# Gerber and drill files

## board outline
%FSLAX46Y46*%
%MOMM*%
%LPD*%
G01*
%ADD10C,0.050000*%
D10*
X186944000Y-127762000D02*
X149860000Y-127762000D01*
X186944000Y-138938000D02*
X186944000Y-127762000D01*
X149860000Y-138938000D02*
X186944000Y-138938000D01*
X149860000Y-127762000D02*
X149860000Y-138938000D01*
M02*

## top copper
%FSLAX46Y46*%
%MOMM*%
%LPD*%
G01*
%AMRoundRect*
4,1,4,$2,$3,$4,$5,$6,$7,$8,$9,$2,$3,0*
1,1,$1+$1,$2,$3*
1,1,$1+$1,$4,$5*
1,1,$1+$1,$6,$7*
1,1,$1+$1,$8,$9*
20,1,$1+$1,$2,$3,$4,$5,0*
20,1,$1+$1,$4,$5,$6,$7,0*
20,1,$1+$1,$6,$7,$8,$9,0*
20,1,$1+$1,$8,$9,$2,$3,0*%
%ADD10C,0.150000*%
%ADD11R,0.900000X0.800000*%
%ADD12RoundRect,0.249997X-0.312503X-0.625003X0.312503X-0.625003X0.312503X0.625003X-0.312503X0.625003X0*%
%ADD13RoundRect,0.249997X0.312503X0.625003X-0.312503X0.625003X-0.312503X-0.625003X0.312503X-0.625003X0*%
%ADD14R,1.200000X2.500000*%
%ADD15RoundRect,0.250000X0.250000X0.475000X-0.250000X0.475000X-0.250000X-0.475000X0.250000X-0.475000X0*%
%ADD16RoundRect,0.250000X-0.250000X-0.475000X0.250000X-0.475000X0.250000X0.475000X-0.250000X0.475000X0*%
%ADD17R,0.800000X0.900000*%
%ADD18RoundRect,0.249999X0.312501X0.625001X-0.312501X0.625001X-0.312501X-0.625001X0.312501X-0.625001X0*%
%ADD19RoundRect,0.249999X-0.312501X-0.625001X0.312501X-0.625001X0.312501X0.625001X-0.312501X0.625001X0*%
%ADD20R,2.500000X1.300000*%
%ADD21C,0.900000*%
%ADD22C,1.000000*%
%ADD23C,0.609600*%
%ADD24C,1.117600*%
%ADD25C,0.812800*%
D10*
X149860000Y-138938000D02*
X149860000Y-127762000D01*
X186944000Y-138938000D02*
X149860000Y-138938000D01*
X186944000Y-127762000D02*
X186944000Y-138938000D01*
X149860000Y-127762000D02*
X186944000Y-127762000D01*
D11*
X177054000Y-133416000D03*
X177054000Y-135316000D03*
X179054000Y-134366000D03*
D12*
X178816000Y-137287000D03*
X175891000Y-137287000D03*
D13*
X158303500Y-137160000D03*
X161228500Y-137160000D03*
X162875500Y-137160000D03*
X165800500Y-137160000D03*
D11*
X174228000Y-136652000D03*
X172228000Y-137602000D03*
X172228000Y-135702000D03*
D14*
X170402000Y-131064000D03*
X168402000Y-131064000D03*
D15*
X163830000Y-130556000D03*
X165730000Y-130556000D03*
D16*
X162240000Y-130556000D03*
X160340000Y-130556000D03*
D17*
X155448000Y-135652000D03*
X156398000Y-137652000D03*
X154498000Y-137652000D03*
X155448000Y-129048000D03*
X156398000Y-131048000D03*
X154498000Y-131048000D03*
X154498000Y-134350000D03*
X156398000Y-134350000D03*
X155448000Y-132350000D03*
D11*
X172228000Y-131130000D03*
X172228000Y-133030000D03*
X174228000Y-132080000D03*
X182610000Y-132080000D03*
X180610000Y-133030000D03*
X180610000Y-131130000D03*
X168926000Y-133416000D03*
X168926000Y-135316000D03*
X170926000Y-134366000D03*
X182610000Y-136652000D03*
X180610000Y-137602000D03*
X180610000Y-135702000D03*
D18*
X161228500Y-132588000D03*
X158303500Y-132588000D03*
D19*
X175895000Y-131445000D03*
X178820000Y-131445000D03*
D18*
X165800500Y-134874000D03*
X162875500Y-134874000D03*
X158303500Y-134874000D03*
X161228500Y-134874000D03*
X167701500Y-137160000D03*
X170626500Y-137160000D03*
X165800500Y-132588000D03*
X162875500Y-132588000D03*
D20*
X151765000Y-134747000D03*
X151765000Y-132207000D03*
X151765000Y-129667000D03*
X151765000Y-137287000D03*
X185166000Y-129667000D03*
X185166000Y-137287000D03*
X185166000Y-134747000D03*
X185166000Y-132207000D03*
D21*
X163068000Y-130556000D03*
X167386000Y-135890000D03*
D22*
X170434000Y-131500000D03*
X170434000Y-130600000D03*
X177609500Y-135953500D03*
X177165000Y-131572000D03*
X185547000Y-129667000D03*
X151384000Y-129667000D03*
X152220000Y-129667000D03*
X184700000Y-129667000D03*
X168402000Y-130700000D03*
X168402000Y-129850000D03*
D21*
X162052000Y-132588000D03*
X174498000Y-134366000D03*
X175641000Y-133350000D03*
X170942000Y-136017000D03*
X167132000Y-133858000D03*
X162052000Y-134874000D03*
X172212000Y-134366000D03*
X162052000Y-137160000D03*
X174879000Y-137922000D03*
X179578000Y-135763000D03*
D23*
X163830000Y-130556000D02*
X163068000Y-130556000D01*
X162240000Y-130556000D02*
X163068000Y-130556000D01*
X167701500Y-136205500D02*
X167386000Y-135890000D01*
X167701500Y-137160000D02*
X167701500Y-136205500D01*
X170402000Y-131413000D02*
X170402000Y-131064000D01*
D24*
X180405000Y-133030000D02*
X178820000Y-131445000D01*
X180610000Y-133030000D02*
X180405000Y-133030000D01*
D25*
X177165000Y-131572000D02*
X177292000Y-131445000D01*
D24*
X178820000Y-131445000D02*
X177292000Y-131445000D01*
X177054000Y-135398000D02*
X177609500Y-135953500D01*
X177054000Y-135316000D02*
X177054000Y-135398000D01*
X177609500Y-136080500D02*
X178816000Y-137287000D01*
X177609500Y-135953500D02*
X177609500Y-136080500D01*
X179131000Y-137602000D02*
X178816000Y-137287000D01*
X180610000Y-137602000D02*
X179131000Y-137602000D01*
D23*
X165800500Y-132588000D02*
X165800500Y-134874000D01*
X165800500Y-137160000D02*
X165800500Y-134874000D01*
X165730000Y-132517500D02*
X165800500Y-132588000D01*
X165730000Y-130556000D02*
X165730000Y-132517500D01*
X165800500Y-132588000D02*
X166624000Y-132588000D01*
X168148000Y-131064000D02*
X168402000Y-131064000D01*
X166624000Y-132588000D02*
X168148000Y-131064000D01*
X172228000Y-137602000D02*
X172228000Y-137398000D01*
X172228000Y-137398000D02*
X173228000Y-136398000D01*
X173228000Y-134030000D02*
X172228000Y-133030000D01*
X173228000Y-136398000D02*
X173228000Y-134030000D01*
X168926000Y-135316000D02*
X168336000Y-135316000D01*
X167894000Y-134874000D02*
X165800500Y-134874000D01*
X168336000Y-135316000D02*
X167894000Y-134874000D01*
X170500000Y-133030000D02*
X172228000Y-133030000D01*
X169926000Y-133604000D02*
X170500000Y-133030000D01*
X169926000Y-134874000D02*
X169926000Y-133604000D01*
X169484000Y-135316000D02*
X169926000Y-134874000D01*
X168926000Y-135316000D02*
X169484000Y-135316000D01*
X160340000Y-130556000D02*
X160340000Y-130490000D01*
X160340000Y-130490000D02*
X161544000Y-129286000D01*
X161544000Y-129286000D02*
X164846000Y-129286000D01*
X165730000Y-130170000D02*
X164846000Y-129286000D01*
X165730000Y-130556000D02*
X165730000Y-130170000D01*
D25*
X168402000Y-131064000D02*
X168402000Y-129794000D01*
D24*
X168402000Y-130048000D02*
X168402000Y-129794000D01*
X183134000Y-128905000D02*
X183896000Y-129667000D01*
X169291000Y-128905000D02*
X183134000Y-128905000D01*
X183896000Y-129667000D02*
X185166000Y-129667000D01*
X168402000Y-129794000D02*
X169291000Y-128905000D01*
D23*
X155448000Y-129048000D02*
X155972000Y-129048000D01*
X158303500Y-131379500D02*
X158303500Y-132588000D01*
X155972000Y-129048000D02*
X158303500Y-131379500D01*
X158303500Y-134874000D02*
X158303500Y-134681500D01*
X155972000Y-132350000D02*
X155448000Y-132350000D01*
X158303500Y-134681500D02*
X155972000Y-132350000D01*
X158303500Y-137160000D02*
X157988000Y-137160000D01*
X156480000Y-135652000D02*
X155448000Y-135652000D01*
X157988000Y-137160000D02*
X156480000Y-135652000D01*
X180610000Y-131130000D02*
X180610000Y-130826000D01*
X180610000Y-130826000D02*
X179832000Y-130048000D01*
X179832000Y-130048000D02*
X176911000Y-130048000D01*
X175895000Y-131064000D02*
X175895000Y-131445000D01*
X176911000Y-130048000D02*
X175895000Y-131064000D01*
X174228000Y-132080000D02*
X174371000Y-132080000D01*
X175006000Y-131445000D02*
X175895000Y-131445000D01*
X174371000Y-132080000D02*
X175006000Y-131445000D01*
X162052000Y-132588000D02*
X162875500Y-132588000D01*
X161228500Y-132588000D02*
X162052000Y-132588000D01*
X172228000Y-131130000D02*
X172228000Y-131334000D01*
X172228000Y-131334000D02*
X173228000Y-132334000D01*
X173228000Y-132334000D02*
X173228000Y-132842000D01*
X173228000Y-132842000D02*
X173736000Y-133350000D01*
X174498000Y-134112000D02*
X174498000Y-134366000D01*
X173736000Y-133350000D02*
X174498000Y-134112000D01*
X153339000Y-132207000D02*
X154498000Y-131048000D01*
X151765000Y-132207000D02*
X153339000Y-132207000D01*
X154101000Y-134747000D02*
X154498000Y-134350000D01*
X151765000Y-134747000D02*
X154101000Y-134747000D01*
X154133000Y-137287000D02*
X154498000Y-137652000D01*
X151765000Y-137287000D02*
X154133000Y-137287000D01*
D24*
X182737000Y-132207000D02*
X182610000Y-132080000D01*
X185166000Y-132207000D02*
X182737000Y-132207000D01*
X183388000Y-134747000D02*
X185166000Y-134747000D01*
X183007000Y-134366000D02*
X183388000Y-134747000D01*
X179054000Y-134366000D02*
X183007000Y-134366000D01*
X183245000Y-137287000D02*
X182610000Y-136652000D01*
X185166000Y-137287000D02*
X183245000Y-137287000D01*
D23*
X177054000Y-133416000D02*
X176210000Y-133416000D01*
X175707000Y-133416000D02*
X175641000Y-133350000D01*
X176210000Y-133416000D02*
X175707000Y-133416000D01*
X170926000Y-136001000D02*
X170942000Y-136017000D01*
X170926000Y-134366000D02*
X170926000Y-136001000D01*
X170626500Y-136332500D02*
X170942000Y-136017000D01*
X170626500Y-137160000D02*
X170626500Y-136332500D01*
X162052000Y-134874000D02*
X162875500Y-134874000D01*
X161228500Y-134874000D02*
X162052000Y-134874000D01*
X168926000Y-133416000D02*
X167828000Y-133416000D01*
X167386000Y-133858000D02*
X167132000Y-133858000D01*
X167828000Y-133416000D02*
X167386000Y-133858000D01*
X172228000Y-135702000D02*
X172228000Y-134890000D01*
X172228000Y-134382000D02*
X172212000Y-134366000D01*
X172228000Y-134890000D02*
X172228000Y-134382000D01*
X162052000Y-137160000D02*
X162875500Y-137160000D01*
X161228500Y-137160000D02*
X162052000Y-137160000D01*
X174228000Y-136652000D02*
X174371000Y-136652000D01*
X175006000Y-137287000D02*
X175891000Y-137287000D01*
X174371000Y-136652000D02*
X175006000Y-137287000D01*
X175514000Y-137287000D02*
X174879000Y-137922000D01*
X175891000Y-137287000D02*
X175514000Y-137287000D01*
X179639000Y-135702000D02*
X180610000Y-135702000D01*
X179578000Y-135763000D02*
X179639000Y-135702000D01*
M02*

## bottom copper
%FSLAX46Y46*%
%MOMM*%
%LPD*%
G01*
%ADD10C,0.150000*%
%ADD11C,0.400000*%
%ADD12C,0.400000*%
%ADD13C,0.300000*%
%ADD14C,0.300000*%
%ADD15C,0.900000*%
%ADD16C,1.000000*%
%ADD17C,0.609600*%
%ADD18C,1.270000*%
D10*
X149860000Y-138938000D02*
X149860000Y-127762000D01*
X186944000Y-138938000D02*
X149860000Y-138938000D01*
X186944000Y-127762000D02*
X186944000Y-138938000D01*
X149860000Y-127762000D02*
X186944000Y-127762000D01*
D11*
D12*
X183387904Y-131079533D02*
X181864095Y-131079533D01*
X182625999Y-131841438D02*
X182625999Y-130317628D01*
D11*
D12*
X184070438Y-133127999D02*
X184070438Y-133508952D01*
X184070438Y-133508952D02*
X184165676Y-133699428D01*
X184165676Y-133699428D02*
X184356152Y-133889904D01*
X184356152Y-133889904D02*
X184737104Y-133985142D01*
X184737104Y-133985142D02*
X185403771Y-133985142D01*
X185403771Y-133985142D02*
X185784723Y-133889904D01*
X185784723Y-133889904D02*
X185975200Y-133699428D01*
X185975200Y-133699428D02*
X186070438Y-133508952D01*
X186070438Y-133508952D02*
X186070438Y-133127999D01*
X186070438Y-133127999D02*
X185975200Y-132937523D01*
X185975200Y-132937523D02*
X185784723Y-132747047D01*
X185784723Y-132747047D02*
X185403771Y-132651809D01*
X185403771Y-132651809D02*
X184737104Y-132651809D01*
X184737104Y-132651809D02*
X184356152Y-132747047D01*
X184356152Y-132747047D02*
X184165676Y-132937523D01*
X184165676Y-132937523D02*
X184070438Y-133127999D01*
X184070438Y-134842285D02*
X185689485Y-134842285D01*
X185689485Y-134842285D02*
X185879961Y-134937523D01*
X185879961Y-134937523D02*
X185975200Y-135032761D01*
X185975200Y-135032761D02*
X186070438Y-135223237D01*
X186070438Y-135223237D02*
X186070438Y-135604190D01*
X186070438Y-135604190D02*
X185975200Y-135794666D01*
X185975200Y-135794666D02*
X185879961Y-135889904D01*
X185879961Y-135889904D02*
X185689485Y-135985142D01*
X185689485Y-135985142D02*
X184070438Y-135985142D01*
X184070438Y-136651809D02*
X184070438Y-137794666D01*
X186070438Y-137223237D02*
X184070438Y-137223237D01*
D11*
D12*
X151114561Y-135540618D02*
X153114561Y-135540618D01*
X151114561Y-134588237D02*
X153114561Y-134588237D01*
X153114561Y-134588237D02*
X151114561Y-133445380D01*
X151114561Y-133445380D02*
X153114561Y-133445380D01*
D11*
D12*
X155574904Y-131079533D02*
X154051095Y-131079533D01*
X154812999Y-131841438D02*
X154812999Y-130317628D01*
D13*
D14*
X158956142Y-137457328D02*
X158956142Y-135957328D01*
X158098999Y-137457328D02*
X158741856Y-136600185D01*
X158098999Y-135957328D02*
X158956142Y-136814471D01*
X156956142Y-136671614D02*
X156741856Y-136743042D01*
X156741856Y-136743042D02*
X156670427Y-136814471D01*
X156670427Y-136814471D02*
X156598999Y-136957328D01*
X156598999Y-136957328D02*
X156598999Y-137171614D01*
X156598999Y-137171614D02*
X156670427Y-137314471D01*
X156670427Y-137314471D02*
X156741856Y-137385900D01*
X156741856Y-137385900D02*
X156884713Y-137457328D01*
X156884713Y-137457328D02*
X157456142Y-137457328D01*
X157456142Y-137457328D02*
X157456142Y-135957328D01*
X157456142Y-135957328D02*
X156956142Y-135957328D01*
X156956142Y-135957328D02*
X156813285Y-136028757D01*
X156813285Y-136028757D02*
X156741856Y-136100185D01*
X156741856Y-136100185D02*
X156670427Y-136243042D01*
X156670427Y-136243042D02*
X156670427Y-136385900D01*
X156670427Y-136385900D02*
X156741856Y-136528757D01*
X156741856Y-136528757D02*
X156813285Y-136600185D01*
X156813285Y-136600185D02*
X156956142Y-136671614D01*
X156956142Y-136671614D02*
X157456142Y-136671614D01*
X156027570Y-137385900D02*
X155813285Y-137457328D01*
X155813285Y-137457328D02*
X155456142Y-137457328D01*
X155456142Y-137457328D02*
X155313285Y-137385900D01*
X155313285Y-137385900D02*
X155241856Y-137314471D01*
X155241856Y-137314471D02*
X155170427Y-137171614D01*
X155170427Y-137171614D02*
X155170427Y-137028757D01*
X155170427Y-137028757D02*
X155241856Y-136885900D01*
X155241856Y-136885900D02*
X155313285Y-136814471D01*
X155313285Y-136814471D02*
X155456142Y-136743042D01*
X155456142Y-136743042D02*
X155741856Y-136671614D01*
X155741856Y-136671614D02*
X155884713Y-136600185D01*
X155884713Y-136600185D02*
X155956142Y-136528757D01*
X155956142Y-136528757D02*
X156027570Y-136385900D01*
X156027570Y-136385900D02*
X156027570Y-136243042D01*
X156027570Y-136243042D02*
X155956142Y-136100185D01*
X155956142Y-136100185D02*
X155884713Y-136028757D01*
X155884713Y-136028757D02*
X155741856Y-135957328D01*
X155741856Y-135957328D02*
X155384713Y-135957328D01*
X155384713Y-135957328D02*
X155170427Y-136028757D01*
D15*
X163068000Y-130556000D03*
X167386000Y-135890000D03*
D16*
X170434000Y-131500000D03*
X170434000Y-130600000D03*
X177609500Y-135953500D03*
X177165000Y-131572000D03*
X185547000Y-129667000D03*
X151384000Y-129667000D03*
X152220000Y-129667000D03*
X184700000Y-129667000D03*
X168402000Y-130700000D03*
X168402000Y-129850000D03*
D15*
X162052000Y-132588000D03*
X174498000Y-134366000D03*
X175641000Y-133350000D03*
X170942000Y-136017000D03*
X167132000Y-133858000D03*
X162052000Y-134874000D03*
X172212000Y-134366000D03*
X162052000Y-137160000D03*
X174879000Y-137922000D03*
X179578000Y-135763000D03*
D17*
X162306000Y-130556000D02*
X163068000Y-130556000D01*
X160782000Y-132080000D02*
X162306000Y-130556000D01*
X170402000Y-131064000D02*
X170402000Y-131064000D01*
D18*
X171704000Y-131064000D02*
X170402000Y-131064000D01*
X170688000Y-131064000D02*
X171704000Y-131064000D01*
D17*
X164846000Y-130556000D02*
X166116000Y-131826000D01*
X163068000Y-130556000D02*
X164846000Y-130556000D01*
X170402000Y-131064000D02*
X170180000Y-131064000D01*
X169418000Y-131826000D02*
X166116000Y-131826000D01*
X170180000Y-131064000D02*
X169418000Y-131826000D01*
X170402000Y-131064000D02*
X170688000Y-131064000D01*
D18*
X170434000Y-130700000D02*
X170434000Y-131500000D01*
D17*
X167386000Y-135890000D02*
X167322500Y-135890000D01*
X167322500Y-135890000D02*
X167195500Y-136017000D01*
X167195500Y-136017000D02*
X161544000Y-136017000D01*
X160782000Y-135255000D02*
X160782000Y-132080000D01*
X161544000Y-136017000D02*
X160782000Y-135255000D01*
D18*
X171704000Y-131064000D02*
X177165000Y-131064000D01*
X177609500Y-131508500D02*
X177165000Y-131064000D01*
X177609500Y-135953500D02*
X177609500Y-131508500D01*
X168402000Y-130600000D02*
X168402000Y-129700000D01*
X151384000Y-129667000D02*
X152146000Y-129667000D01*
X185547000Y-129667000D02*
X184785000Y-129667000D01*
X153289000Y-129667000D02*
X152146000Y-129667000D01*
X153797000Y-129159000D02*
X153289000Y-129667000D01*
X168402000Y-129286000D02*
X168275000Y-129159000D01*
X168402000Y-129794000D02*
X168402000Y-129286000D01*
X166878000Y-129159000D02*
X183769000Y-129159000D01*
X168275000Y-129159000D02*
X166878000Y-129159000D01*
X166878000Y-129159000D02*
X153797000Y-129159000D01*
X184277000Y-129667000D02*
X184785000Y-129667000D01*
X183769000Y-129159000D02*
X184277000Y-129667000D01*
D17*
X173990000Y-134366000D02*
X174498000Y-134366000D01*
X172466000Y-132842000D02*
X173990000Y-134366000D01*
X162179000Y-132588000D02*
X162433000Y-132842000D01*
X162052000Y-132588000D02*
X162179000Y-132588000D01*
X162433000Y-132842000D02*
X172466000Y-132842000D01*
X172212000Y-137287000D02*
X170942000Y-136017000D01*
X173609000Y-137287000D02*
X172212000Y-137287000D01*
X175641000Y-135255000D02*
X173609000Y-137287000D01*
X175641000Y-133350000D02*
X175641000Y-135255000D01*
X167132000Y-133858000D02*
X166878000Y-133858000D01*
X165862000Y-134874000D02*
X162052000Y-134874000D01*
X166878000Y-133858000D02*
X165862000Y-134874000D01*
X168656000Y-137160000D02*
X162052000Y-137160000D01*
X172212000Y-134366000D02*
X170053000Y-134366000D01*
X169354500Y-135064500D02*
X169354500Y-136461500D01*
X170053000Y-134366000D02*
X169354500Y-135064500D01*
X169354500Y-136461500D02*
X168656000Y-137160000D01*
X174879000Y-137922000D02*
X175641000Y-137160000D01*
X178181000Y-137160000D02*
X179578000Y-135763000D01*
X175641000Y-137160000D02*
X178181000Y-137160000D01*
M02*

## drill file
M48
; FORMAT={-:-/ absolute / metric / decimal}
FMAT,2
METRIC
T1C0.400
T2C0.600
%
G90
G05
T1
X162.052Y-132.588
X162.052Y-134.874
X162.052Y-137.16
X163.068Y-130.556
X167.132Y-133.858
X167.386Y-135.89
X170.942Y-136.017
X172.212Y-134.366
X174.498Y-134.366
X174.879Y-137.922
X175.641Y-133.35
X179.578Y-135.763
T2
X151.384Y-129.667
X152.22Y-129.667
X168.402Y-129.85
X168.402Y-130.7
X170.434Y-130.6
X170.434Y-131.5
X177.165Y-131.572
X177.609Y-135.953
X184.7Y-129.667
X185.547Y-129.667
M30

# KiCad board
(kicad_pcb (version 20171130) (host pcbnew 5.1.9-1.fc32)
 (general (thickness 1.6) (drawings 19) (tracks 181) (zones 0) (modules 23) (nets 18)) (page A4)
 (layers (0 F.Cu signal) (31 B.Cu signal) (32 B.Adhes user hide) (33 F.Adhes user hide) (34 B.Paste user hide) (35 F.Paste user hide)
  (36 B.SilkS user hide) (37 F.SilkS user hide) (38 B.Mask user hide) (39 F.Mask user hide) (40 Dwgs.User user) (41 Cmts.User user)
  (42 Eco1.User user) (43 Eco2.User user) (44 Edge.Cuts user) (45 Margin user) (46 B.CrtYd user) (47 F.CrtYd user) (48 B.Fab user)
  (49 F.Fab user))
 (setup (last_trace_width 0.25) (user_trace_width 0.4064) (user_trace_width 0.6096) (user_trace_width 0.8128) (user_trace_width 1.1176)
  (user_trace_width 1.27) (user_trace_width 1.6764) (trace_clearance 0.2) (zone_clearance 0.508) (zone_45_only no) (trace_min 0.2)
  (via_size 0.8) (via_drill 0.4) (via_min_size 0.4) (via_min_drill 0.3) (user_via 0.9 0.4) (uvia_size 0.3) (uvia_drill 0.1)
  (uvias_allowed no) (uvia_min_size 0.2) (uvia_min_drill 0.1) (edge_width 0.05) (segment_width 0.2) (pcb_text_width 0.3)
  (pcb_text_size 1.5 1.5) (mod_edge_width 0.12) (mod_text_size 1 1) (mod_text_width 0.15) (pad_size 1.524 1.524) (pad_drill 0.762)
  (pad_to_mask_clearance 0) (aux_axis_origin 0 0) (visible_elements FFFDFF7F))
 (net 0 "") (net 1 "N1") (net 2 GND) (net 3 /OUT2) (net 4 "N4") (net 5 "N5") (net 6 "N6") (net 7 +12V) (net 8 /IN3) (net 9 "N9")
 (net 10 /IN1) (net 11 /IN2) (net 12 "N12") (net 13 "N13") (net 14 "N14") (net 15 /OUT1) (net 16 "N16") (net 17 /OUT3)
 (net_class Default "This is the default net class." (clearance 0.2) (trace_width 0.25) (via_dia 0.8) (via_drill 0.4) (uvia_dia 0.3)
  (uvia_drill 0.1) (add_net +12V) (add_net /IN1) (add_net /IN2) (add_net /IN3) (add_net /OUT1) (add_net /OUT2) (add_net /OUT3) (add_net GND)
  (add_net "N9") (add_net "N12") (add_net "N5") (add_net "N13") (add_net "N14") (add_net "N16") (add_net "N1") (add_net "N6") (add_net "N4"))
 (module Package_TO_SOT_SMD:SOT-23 (layer F.Cu) (at 178.054 134.366)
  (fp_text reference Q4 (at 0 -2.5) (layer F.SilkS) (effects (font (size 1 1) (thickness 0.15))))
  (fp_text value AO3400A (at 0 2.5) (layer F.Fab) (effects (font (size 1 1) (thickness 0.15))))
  (pad 1 smd rect (at -1 -0.95) (size 0.9 0.8) (layers F.Cu F.Paste F.Mask) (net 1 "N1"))
  (pad 2 smd rect (at -1 0.95) (size 0.9 0.8) (layers F.Cu F.Paste F.Mask) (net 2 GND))
  (pad 3 smd rect (at 1 0) (size 0.9 0.8) (layers F.Cu F.Paste F.Mask) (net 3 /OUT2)))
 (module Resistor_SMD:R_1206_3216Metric (layer F.Cu) (at 177.3535 137.287)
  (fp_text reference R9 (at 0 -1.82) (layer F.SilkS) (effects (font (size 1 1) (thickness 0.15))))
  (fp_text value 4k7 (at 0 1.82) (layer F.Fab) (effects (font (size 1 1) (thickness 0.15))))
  (pad 2 smd roundrect (at 1.4625 0) (size 1.125 1.75) (layers F.Cu F.Paste F.Mask) (roundrect_rratio 0.2222195555555556) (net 2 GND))
  (pad 1 smd roundrect (at -1.4625 0) (size 1.125 1.75) (layers F.Cu F.Paste F.Mask) (roundrect_rratio 0.2222195555555556) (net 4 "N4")))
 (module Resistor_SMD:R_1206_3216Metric (layer F.Cu) (at 159.766 137.16 180)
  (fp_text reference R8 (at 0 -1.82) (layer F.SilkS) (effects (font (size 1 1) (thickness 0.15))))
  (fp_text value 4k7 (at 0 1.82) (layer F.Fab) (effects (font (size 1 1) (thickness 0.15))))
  (pad 2 smd roundrect (at 1.4625 0 180) (size 1.125 1.75) (layers F.Cu F.Paste F.Mask) (roundrect_rratio 0.2222195555555556) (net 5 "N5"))
  (pad 1 smd roundrect (at -1.4625 0 180) (size 1.125 1.75) (layers F.Cu F.Paste F.Mask) (roundrect_rratio 0.2222195555555556) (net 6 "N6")))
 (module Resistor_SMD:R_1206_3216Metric (layer F.Cu) (at 164.338 137.16 180)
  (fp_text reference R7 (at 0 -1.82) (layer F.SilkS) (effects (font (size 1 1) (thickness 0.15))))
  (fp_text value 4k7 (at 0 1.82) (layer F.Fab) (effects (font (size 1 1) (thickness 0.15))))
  (pad 2 smd roundrect (at 1.4625 0 180) (size 1.125 1.75) (layers F.Cu F.Paste F.Mask) (roundrect_rratio 0.2222195555555556) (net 6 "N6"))
  (pad 1 smd roundrect (at -1.4625 0 180) (size 1.125 1.75) (layers F.Cu F.Paste F.Mask) (roundrect_rratio 0.2222195555555556) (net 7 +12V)))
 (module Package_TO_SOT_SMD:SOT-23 (layer F.Cu) (at 173.228 136.652)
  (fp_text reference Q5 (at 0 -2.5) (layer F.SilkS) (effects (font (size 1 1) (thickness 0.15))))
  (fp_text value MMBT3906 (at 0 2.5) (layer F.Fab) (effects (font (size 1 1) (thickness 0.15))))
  (pad 3 smd rect (at 1 0) (size 0.9 0.8) (layers F.Cu F.Paste F.Mask) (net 4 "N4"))
  (pad 2 smd rect (at -1 0.95) (size 0.9 0.8) (layers F.Cu F.Paste F.Mask) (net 7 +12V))
  (pad 1 smd rect (at -1 -0.95) (size 0.9 0.8) (layers F.Cu F.Paste F.Mask) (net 6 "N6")))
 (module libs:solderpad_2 (layer F.Cu) (at 168.402 131.064)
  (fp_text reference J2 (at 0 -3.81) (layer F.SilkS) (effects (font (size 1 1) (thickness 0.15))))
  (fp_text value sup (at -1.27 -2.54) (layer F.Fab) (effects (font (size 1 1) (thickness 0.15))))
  (pad 2 smd rect (at 2 0 90) (size 2.5 1.2) (layers F.Cu F.Paste F.Mask) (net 2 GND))
  (pad 1 smd rect (at 0 0 90) (size 2.5 1.2) (layers F.Cu F.Paste F.Mask) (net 7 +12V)))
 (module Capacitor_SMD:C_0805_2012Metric (layer F.Cu) (at 164.78 130.556 180)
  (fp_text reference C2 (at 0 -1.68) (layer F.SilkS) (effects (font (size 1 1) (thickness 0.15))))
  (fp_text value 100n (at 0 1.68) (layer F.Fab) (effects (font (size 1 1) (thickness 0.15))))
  (pad 2 smd roundrect (at 0.95 0 180) (size 1 1.45) (layers F.Cu F.Paste F.Mask) (roundrect_rratio 0.25) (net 2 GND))
  (pad 1 smd roundrect (at -0.95 0 180) (size 1 1.45) (layers F.Cu F.Paste F.Mask) (roundrect_rratio 0.25) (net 7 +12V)))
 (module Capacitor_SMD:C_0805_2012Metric (layer F.Cu) (at 161.29 130.556)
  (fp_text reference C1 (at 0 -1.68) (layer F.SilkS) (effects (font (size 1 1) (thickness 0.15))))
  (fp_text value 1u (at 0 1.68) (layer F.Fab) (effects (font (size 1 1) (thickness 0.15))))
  (pad 2 smd roundrect (at 0.95 0) (size 1 1.45) (layers F.Cu F.Paste F.Mask) (roundrect_rratio 0.25) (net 2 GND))
  (pad 1 smd roundrect (at -0.95 0) (size 1 1.45) (layers F.Cu F.Paste F.Mask) (roundrect_rratio 0.25) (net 7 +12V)))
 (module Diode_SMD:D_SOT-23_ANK (layer F.Cu) (at 155.448 136.652 90)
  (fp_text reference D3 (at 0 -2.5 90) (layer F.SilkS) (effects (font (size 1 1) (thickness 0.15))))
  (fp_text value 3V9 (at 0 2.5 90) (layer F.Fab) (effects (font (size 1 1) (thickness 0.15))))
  (pad 1 smd rect (at 1 0 90) (size 0.9 0.8) (layers F.Cu F.Paste F.Mask) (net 5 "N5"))
  (pad "" smd rect (at -1 0.95 90) (size 0.9 0.8) (layers F.Cu F.Paste F.Mask))
  (pad 2 smd rect (at -1 -0.95 90) (size 0.9 0.8) (layers F.Cu F.Paste F.Mask) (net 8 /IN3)))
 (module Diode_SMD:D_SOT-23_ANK (layer F.Cu) (at 155.448 130.048 90)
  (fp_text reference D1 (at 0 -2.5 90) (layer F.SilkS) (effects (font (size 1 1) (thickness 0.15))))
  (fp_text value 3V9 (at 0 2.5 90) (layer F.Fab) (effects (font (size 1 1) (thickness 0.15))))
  (pad 1 smd rect (at 1 0 90) (size 0.9 0.8) (layers F.Cu F.Paste F.Mask) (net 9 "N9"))
  (pad "" smd rect (at -1 0.95 90) (size 0.9 0.8) (layers F.Cu F.Paste F.Mask))
  (pad 2 smd rect (at -1 -0.95 90) (size 0.9 0.8) (layers F.Cu F.Paste F.Mask) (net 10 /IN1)))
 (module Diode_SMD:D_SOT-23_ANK (layer F.Cu) (at 155.448 133.35 90)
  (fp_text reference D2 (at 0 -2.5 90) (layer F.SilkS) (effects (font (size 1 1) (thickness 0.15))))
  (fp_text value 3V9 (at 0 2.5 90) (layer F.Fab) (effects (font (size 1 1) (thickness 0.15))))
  (pad 2 smd rect (at -1 -0.95 90) (size 0.9 0.8) (layers F.Cu F.Paste F.Mask) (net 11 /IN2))
  (pad "" smd rect (at -1 0.95 90) (size 0.9 0.8) (layers F.Cu F.Paste F.Mask))
  (pad 1 smd rect (at 1 0 90) (size 0.9 0.8) (layers F.Cu F.Paste F.Mask) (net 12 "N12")))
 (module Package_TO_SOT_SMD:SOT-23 (layer F.Cu) (at 173.228 132.08)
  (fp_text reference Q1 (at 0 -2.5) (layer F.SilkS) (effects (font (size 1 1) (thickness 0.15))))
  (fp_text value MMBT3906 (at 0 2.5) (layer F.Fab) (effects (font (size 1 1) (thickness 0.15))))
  (pad 1 smd rect (at -1 -0.95) (size 0.9 0.8) (layers F.Cu F.Paste F.Mask) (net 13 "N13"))
  (pad 2 smd rect (at -1 0.95) (size 0.9 0.8) (layers F.Cu F.Paste F.Mask) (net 7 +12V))
  (pad 3 smd rect (at 1 0) (size 0.9 0.8) (layers F.Cu F.Paste F.Mask) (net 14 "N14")))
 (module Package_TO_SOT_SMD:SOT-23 (layer F.Cu) (at 181.61 132.08)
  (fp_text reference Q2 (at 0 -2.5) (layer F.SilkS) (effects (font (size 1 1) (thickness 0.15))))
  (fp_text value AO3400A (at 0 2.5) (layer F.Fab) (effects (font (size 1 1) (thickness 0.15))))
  (pad 3 smd rect (at 1 0) (size 0.9 0.8) (layers F.Cu F.Paste F.Mask) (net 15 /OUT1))
  (pad 2 smd rect (at -1 0.95) (size 0.9 0.8) (layers F.Cu F.Paste F.Mask) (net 2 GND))
  (pad 1 smd rect (at -1 -0.95) (size 0.9 0.8) (layers F.Cu F.Paste F.Mask) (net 14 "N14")))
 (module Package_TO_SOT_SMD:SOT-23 (layer F.Cu) (at 169.926 134.366)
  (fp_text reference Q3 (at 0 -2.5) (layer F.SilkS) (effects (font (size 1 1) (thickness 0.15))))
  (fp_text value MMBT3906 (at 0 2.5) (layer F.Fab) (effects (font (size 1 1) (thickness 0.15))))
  (pad 1 smd rect (at -1 -0.95) (size 0.9 0.8) (layers F.Cu F.Paste F.Mask) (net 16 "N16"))
  (pad 2 smd rect (at -1 0.95) (size 0.9 0.8) (layers F.Cu F.Paste F.Mask) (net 7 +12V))
  (pad 3 smd rect (at 1 0) (size 0.9 0.8) (layers F.Cu F.Paste F.Mask) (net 1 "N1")))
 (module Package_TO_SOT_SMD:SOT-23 (layer F.Cu) (at 181.61 136.652)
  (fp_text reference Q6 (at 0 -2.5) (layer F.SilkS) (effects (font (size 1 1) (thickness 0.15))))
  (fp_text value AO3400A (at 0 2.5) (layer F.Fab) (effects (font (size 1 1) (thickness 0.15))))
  (pad 3 smd rect (at 1 0) (size 0.9 0.8) (layers F.Cu F.Paste F.Mask) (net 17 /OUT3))
  (pad 2 smd rect (at -1 0.95) (size 0.9 0.8) (layers F.Cu F.Paste F.Mask) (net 2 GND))
  (pad 1 smd rect (at -1 -0.95) (size 0.9 0.8) (layers F.Cu F.Paste F.Mask) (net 4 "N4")))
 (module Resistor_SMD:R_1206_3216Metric (layer F.Cu) (at 159.766 132.588 180)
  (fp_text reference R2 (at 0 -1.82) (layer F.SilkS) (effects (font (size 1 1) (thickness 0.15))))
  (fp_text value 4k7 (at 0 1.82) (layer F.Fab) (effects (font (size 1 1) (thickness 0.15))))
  (pad 1 smd roundrect (at -1.4625 0 180) (size 1.125 1.75) (layers F.Cu F.Paste F.Mask) (roundrect_rratio 0.2222213333333333)
   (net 13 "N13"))
  (pad 2 smd roundrect (at 1.4625 0 180) (size 1.125 1.75) (layers F.Cu F.Paste F.Mask) (roundrect_rratio 0.2222213333333333) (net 9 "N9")))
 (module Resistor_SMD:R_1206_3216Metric (layer F.Cu) (at 177.3575 131.445)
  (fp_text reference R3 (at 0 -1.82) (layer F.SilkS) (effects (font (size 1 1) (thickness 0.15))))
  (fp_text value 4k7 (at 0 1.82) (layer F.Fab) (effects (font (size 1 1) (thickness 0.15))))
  (pad 1 smd roundrect (at -1.4625 0) (size 1.125 1.75) (layers F.Cu F.Paste F.Mask) (roundrect_rratio 0.2222213333333333) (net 14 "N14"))
  (pad 2 smd roundrect (at 1.4625 0) (size 1.125 1.75) (layers F.Cu F.Paste F.Mask) (roundrect_rratio 0.2222213333333333) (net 2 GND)))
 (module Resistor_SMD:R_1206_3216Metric (layer F.Cu) (at 164.338 134.874 180)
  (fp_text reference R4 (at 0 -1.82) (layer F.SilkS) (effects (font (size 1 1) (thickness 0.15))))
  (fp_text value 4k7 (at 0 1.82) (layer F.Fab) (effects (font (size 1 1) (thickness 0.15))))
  (pad 1 smd roundrect (at -1.4625 0 180) (size 1.125 1.75) (layers F.Cu F.Paste F.Mask) (roundrect_rratio 0.2222213333333333) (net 7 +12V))
  (pad 2 smd roundrect (at 1.4625 0 180) (size 1.125 1.75) (layers F.Cu F.Paste F.Mask) (roundrect_rratio 0.2222213333333333) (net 16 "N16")))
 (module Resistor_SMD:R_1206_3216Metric (layer F.Cu) (at 159.766 134.874 180)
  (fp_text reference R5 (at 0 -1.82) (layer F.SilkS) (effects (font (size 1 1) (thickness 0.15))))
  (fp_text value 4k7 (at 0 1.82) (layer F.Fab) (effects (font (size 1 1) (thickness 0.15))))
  (pad 2 smd roundrect (at 1.4625 0 180) (size 1.125 1.75) (layers F.Cu F.Paste F.Mask) (roundrect_rratio 0.2222213333333333) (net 12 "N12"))
  (pad 1 smd roundrect (at -1.4625 0 180) (size 1.125 1.75) (layers F.Cu F.Paste F.Mask) (roundrect_rratio 0.2222213333333333)
   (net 16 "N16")))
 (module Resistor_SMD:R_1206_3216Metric (layer F.Cu) (at 169.164 137.16 180)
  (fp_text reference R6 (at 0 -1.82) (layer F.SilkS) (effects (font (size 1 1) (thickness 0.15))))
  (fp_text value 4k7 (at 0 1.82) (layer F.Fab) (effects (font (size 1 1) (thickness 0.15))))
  (pad 2 smd roundrect (at 1.4625 0 180) (size 1.125 1.75) (layers F.Cu F.Paste F.Mask) (roundrect_rratio 0.2222213333333333) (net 2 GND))
  (pad 1 smd roundrect (at -1.4625 0 180) (size 1.125 1.75) (layers F.Cu F.Paste F.Mask) (roundrect_rratio 0.2222213333333333) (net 1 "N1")))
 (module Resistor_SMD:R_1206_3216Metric (layer F.Cu) (at 164.338 132.588 180)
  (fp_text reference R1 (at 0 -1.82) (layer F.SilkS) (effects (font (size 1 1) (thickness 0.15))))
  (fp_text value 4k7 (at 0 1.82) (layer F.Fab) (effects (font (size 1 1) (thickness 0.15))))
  (pad 1 smd roundrect (at -1.4625 0 180) (size 1.125 1.75) (layers F.Cu F.Paste F.Mask) (roundrect_rratio 0.2222213333333333) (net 7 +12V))
  (pad 2 smd roundrect (at 1.4625 0 180) (size 1.125 1.75) (layers F.Cu F.Paste F.Mask) (roundrect_rratio 0.2222213333333333) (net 13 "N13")))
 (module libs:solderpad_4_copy (layer F.Cu) (at 151.765 129.667 270)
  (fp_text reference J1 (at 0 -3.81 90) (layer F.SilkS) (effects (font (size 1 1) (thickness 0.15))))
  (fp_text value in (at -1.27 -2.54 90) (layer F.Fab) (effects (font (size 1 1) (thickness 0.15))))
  (pad 3 smd rect (at 5.08 0) (size 2.5 1.3) (layers F.Cu F.Paste F.Mask) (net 11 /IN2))
  (pad 2 smd rect (at 2.54 0) (size 2.5 1.3) (layers F.Cu F.Paste F.Mask) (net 10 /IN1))
  (pad 1 smd rect (at 0 0) (size 2.5 1.3) (layers F.Cu F.Paste F.Mask) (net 7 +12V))
  (pad 4 smd rect (at 7.62 0) (size 2.5 1.3) (layers F.Cu F.Paste F.Mask) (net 8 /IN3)))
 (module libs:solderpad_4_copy (layer F.Cu) (at 185.166 137.287 90)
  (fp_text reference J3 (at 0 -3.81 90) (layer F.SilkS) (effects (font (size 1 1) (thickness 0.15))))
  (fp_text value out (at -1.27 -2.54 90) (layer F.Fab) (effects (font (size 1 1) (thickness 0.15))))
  (pad 4 smd rect (at 7.62 0 180) (size 2.5 1.3) (layers F.Cu F.Paste F.Mask) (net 7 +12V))
  (pad 1 smd rect (at 0 0 180) (size 2.5 1.3) (layers F.Cu F.Paste F.Mask) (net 17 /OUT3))
  (pad 2 smd rect (at 2.54 0 180) (size 2.5 1.3) (layers F.Cu F.Paste F.Mask) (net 3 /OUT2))
  (pad 3 smd rect (at 5.08 0 180) (size 2.5 1.3) (layers F.Cu F.Paste F.Mask) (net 15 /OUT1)))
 (gr_line (start 186.944 127.762) (end 149.86 127.762) (layer Edge.Cuts) (width 0.05))
 (gr_line (start 186.944 138.938) (end 186.944 127.762) (layer Edge.Cuts) (width 0.05))
 (gr_line (start 149.86 138.938) (end 186.944 138.938) (layer Edge.Cuts) (width 0.05))
 (gr_line (start 149.86 127.762) (end 149.86 138.938) (layer Edge.Cuts) (width 0.05))
 (gr_line (start 149.86 138.938) (end 149.86 127.762) (layer B.Cu) (width 0.15))
 (gr_line (start 186.944 138.938) (end 149.86 138.938) (layer B.Cu) (width 0.15))
 (gr_line (start 186.944 127.762) (end 186.944 138.938) (layer B.Cu) (width 0.15))
 (gr_line (start 149.86 127.762) (end 186.944 127.762) (layer B.Cu) (width 0.15))
 (gr_line (start 149.86 138.938) (end 149.86 127.762) (layer F.Cu) (width 0.15))
 (gr_line (start 186.944 138.938) (end 149.86 138.938) (layer F.Cu) (width 0.15))
 (gr_line (start 186.944 127.762) (end 186.944 138.938) (layer F.Cu) (width 0.15))
 (gr_line (start 149.86 127.762) (end 186.944 127.762) (layer F.Cu) (width 0.15))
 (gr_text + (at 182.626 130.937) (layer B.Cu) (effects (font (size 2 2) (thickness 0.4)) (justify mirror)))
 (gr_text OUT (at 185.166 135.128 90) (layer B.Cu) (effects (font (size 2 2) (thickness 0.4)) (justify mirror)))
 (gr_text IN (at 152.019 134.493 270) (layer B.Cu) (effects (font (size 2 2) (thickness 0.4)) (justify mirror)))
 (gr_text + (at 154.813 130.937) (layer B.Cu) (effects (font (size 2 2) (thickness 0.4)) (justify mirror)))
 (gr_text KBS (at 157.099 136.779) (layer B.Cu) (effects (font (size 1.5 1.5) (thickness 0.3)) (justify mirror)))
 (via (at 163.068 130.556) (size 0.9) (drill 0.4) (layers F.Cu B.Cu) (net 2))
 (segment (start 163.83 130.556) (end 163.068 130.556) (width 0.6096) (layer F.Cu) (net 2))
 (segment (start 162.24 130.556) (end 163.068 130.556) (width 0.6096) (layer F.Cu) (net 2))
 (via (at 167.386 135.89) (size 0.9) (drill 0.4) (layers F.Cu B.Cu) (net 2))
 (segment (start 167.7015 136.2055) (end 167.386 135.89) (width 0.6096) (layer F.Cu) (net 2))
 (segment (start 167.7015 137.16) (end 167.7015 136.2055) (width 0.6096) (layer F.Cu) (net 2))
 (segment (start 162.306 130.556) (end 163.068 130.556) (width 0.6096) (layer B.Cu) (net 2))
 (segment (start 160.782 132.08) (end 162.306 130.556) (width 0.6096) (layer B.Cu) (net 2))
 (via (at 170.434 131.5) (size 1) (drill 0.6) (layers F.Cu B.Cu) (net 2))
 (segment (start 170.402 131.413) (end 170.402 131.064) (width 0.6096) (layer F.Cu) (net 2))
 (segment (start 170.402 131.064) (end 170.402 131.064) (width 0.6096) (layer B.Cu) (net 2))
 (segment (start 171.704 131.064) (end 170.402 131.064) (width 1.27) (layer B.Cu) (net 2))
 (segment (start 170.688 131.064) (end 171.704 131.064) (width 1.27) (layer B.Cu) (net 2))
 (segment (start 164.846 130.556) (end 166.116 131.826) (width 0.6096) (layer B.Cu) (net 2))
 (segment (start 163.068 130.556) (end 164.846 130.556) (width 0.6096) (layer B.Cu) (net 2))
 (segment (start 170.402 131.064) (end 170.18 131.064) (width 0.6096) (layer B.Cu) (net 2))
 (segment (start 169.418 131.826) (end 166.116 131.826) (width 0.6096) (layer B.Cu) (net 2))
 (segment (start 170.18 131.064) (end 169.418 131.826) (width 0.6096) (layer B.Cu) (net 2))
 (segment (start 170.402 131.064) (end 170.688 131.064) (width 0.6096) (layer B.Cu) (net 2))
 (via (at 170.434 130.6) (size 1) (drill 0.6) (layers F.Cu B.Cu) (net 2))
 (segment (start 170.434 130.7) (end 170.434 131.5) (width 1.27) (layer B.Cu) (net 2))
 (segment (start 167.386 135.89) (end 167.3225 135.89) (width 0.6096) (layer B.Cu) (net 2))
 (segment (start 167.3225 135.89) (end 167.1955 136.017) (width 0.6096) (layer B.Cu) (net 2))
 (segment (start 167.1955 136.017) (end 161.544 136.017) (width 0.6096) (layer B.Cu) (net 2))
 (segment (start 160.782 135.255) (end 160.782 132.08) (width 0.6096) (layer B.Cu) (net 2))
 (segment (start 161.544 136.017) (end 160.782 135.255) (width 0.6096) (layer B.Cu) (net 2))
 (segment (start 171.704 131.064) (end 177.165 131.064) (width 1.27) (layer B.Cu) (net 2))
 (via (at 177.6095 135.9535) (size 1) (drill 0.6) (layers F.Cu B.Cu) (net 2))
 (segment (start 177.6095 131.5085) (end 177.165 131.064) (width 1.27) (layer B.Cu) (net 2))
 (segment (start 177.6095 135.9535) (end 177.6095 131.5085) (width 1.27) (layer B.Cu) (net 2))
 (via (at 177.165 131.572) (size 1) (drill 0.6) (layers F.Cu B.Cu) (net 2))
 (segment (start 180.405 133.03) (end 178.82 131.445) (width 1.1176) (layer F.Cu) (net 2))
 (segment (start 180.61 133.03) (end 180.405 133.03) (width 1.1176) (layer F.Cu) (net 2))
 (segment (start 177.165 131.572) (end 177.292 131.445) (width 0.8128) (layer F.Cu) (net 2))
 (segment (start 178.82 131.445) (end 177.292 131.445) (width 1.1176) (layer F.Cu) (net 2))
 (segment (start 177.054 135.398) (end 177.6095 135.9535) (width 1.1176) (layer F.Cu) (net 2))
 (segment (start 177.054 135.316) (end 177.054 135.398) (width 1.1176) (layer F.Cu) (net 2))
 (segment (start 177.6095 136.0805) (end 178.816 137.287) (width 1.1176) (layer F.Cu) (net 2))
 (segment (start 177.6095 135.9535) (end 177.6095 136.0805) (width 1.1176) (layer F.Cu) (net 2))
 (segment (start 179.131 137.602) (end 178.816 137.287) (width 1.1176) (layer F.Cu) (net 2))
 (segment (start 180.61 137.602) (end 179.131 137.602) (width 1.1176) (layer F.Cu) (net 2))
 (via (at 185.547 129.667) (size 1) (drill 0.6) (layers F.Cu B.Cu) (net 7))
 (via (at 151.384 129.667) (size 1) (drill 0.6) (layers F.Cu B.Cu) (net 7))
 (segment (start 165.8005 132.588) (end 165.8005 134.874) (width 0.6096) (layer F.Cu) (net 7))
 (segment (start 165.8005 137.16) (end 165.8005 134.874) (width 0.6096) (layer F.Cu) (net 7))
 (segment (start 165.73 132.5175) (end 165.8005 132.588) (width 0.6096) (layer F.Cu) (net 7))
 (segment (start 165.73 130.556) (end 165.73 132.5175) (width 0.6096) (layer F.Cu) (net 7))
 (segment (start 165.8005 132.588) (end 166.624 132.588) (width 0.6096) (layer F.Cu) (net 7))
 (segment (start 168.148 131.064) (end 168.402 131.064) (width 0.6096) (layer F.Cu) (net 7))
 (segment (start 166.624 132.588) (end 168.148 131.064) (width 0.6096) (layer F.Cu) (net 7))
 (segment (start 172.228 137.602) (end 172.228 137.398) (width 0.6096) (layer F.Cu) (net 7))
 (segment (start 172.228 137.398) (end 173.228 136.398) (width 0.6096) (layer F.Cu) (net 7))
 (segment (start 173.228 134.03) (end 172.228 133.03) (width 0.6096) (layer F.Cu) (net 7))
 (segment (start 173.228 136.398) (end 173.228 134.03) (width 0.6096) (layer F.Cu) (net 7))
 (segment (start 168.926 135.316) (end 168.336 135.316) (width 0.6096) (layer F.Cu) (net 7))
 (segment (start 167.894 134.874) (end 165.8005 134.874) (width 0.6096) (layer F.Cu) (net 7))
 (segment (start 168.336 135.316) (end 167.894 134.874) (width 0.6096) (layer F.Cu) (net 7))
 (segment (start 170.5 133.03) (end 172.228 133.03) (width 0.6096) (layer F.Cu) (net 7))
 (segment (start 169.926 133.604) (end 170.5 133.03) (width 0.6096) (layer F.Cu) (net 7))
 (segment (start 169.926 134.874) (end 169.926 133.604) (width 0.6096) (layer F.Cu) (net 7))
 (segment (start 169.484 135.316) (end 169.926 134.874) (width 0.6096) (layer F.Cu) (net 7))
 (segment (start 168.926 135.316) (end 169.484 135.316) (width 0.6096) (layer F.Cu) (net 7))
 (segment (start 160.34 130.556) (end 160.34 130.49) (width 0.6096) (layer F.Cu) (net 7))
 (segment (start 160.34 130.49) (end 161.544 129.286) (width 0.6096) (layer F.Cu) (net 7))
 (segment (start 161.544 129.286) (end 164.846 129.286) (width 0.6096) (layer F.Cu) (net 7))
 (segment (start 165.73 130.17) (end 164.846 129.286) (width 0.6096) (layer F.Cu) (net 7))
 (segment (start 165.73 130.556) (end 165.73 130.17) (width 0.6096) (layer F.Cu) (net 7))
 (segment (start 168.402 131.064) (end 168.402 129.794) (width 0.8128) (layer F.Cu) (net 7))
 (via (at 152.22 129.667) (size 1) (drill 0.6) (layers F.Cu B.Cu) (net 7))
 (via (at 184.7 129.667) (size 1) (drill 0.6) (layers F.Cu B.Cu) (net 7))
 (via (at 168.402 130.7) (size 1) (drill 0.6) (layers F.Cu B.Cu) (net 7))
 (segment (start 168.402 130.6) (end 168.402 129.7) (width 1.27) (layer B.Cu) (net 7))
 (via (at 168.402 129.85) (size 1) (drill 0.6) (layers F.Cu B.Cu) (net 7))
 (segment (start 151.384 129.667) (end 152.146 129.667) (width 1.27) (layer B.Cu) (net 7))
 (segment (start 168.402 130.048) (end 168.402 129.794) (width 1.1176) (layer F.Cu) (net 7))
 (segment (start 185.547 129.667) (end 184.785 129.667) (width 1.27) (layer B.Cu) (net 7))
 (segment (start 183.134 128.905) (end 183.896 129.667) (width 1.1176) (layer F.Cu) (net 7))
 (segment (start 169.291 128.905) (end 183.134 128.905) (width 1.1176) (layer F.Cu) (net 7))
 (segment (start 183.896 129.667) (end 185.166 129.667) (width 1.1176) (layer F.Cu) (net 7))
 (segment (start 168.402 129.794) (end 169.291 128.905) (width 1.1176) (layer F.Cu) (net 7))
 (segment (start 153.289 129.667) (end 152.146 129.667) (width 1.27) (layer B.Cu) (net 7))
 (segment (start 153.797 129.159) (end 153.289 129.667) (width 1.27) (layer B.Cu) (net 7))
 (segment (start 168.402 129.286) (end 168.275 129.159) (width 1.27) (layer B.Cu) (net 7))
 (segment (start 168.402 129.794) (end 168.402 129.286) (width 1.27) (layer B.Cu) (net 7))
 (segment (start 166.878 129.159) (end 183.769 129.159) (width 1.27) (layer B.Cu) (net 7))
 (segment (start 168.275 129.159) (end 166.878 129.159) (width 1.27) (layer B.Cu) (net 7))
 (segment (start 166.878 129.159) (end 153.797 129.159) (width 1.27) (layer B.Cu) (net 7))
 (segment (start 184.277 129.667) (end 184.785 129.667) (width 1.27) (layer B.Cu) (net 7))
 (segment (start 183.769 129.159) (end 184.277 129.667) (width 1.27) (layer B.Cu) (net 7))
 (segment (start 155.448 129.048) (end 155.972 129.048) (width 0.6096) (layer F.Cu) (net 9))
 (segment (start 158.3035 131.3795) (end 158.3035 132.588) (width 0.6096) (layer F.Cu) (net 9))
 (segment (start 155.972 129.048) (end 158.3035 131.3795) (width 0.6096) (layer F.Cu) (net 9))
 (segment (start 158.3035 134.874) (end 158.3035 134.6815) (width 0.6096) (layer F.Cu) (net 12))
 (segment (start 155.972 132.35) (end 155.448 132.35) (width 0.6096) (layer F.Cu) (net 12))
 (segment (start 158.3035 134.6815) (end 155.972 132.35) (width 0.6096) (layer F.Cu) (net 12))
 (segment (start 158.3035 137.16) (end 157.988 137.16) (width 0.6096) (layer F.Cu) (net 5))
 (segment (start 156.48 135.652) (end 155.448 135.652) (width 0.6096) (layer F.Cu) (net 5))
 (segment (start 157.988 137.16) (end 156.48 135.652) (width 0.6096) (layer F.Cu) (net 5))
 (segment (start 180.61 131.13) (end 180.61 130.826) (width 0.6096) (layer F.Cu) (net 14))
 (segment (start 180.61 130.826) (end 179.832 130.048) (width 0.6096) (layer F.Cu) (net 14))
 (segment (start 179.832 130.048) (end 176.911 130.048) (width 0.6096) (layer F.Cu) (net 14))
 (segment (start 175.895 131.064) (end 175.895 131.445) (width 0.6096) (layer F.Cu) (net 14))
 (segment (start 176.911 130.048) (end 175.895 131.064) (width 0.6096) (layer F.Cu) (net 14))
 (segment (start 174.228 132.08) (end 174.371 132.08) (width 0.6096) (layer F.Cu) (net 14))
 (segment (start 175.006 131.445) (end 175.895 131.445) (width 0.6096) (layer F.Cu) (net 14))
 (segment (start 174.371 132.08) (end 175.006 131.445) (width 0.6096) (layer F.Cu) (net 14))
 (via (at 162.052 132.588) (size 0.9) (drill 0.4) (layers F.Cu B.Cu) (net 13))
 (segment (start 162.052 132.588) (end 162.8755 132.588) (width 0.6096) (layer F.Cu) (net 13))
 (segment (start 161.2285 132.588) (end 162.052 132.588) (width 0.6096) (layer F.Cu) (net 13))
 (segment (start 172.228 131.13) (end 172.228 131.334) (width 0.6096) (layer F.Cu) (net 13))
 (segment (start 172.228 131.334) (end 173.228 132.334) (width 0.6096) (layer F.Cu) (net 13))
 (segment (start 173.228 132.334) (end 173.228 132.842) (width 0.6096) (layer F.Cu) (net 13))
 (segment (start 173.228 132.842) (end 173.736 133.35) (width 0.6096) (layer F.Cu) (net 13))
 (via (at 174.498 134.366) (size 0.9) (drill 0.4) (layers F.Cu B.Cu) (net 13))
 (segment (start 174.498 134.112) (end 174.498 134.366) (width 0.6096) (layer F.Cu) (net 13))
 (segment (start 173.736 133.35) (end 174.498 134.112) (width 0.6096) (layer F.Cu) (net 13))
 (segment (start 173.99 134.366) (end 174.498 134.366) (width 0.6096) (layer B.Cu) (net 13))
 (segment (start 172.466 132.842) (end 173.99 134.366) (width 0.6096) (layer B.Cu) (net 13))
 (segment (start 162.179 132.588) (end 162.433 132.842) (width 0.6096) (layer B.Cu) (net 13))
 (segment (start 162.052 132.588) (end 162.179 132.588) (width 0.6096) (layer B.Cu) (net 13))
 (segment (start 162.433 132.842) (end 172.466 132.842) (width 0.6096) (layer B.Cu) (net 13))
 (segment (start 153.339 132.207) (end 154.498 131.048) (width 0.6096) (layer F.Cu) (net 10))
 (segment (start 151.765 132.207) (end 153.339 132.207) (width 0.6096) (layer F.Cu) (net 10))
 (segment (start 154.101 134.747) (end 154.498 134.35) (width 0.6096) (layer F.Cu) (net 11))
 (segment (start 151.765 134.747) (end 154.101 134.747) (width 0.6096) (layer F.Cu) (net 11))
 (segment (start 154.133 137.287) (end 154.498 137.652) (width 0.6096) (layer F.Cu) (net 8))
 (segment (start 151.765 137.287) (end 154.133 137.287) (width 0.6096) (layer F.Cu) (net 8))
 (segment (start 182.737 132.207) (end 182.61 132.08) (width 1.1176) (layer F.Cu) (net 15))
 (segment (start 185.166 132.207) (end 182.737 132.207) (width 1.1176) (layer F.Cu) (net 15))
 (segment (start 183.388 134.747) (end 185.166 134.747) (width 1.1176) (layer F.Cu) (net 3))
 (segment (start 183.007 134.366) (end 183.388 134.747) (width 1.1176) (layer F.Cu) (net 3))
 (segment (start 179.054 134.366) (end 183.007 134.366) (width 1.1176) (layer F.Cu) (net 3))
 (segment (start 183.245 137.287) (end 182.61 136.652) (width 1.1176) (layer F.Cu) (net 17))
 (segment (start 185.166 137.287) (end 183.245 137.287) (width 1.1176) (layer F.Cu) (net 17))
 (segment (start 177.054 133.416) (end 176.21 133.416) (width 0.6096) (layer F.Cu) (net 1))
 (via (at 175.641 133.35) (size 0.9) (drill 0.4) (layers F.Cu B.Cu) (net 1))
 (segment (start 175.707 133.416) (end 175.641 133.35) (width 0.6096) (layer F.Cu) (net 1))
 (segment (start 176.21 133.416) (end 175.707 133.416) (width 0.6096) (layer F.Cu) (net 1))
 (segment (start 172.212 137.287) (end 170.942 136.017) (width 0.6096) (layer B.Cu) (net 1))
 (via (at 170.942 136.017) (size 0.9) (drill 0.4) (layers F.Cu B.Cu) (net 1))
 (segment (start 173.609 137.287) (end 172.212 137.287) (width 0.6096) (layer B.Cu) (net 1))
 (segment (start 175.641 135.255) (end 173.609 137.287) (width 0.6096) (layer B.Cu) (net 1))
 (segment (start 175.641 133.35) (end 175.641 135.255) (width 0.6096) (layer B.Cu) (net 1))
 (segment (start 170.926 136.001) (end 170.942 136.017) (width 0.6096) (layer F.Cu) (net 1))
 (segment (start 170.926 134.366) (end 170.926 136.001) (width 0.6096) (layer F.Cu) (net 1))
 (segment (start 170.6265 136.3325) (end 170.942 136.017) (width 0.6096) (layer F.Cu) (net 1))
 (segment (start 170.6265 137.16) (end 170.6265 136.3325) (width 0.6096) (layer F.Cu) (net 1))
 (segment (start 162.052 134.874) (end 162.8755 134.874) (width 0.6096) (layer F.Cu) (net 16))
 (segment (start 161.2285 134.874) (end 162.052 134.874) (width 0.6096) (layer F.Cu) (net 16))
 (segment (start 168.926 133.416) (end 167.828 133.416) (width 0.6096) (layer F.Cu) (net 16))
 (via (at 167.132 133.858) (size 0.9) (drill 0.4) (layers F.Cu B.Cu) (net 16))
 (segment (start 167.386 133.858) (end 167.132 133.858) (width 0.6096) (layer F.Cu) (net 16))
 (segment (start 167.828 133.416) (end 167.386 133.858) (width 0.6096) (layer F.Cu) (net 16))
 (segment (start 167.132 133.858) (end 166.878 133.858) (width 0.6096) (layer B.Cu) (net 16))
 (segment (start 165.862 134.874) (end 162.052 134.874) (width 0.6096) (layer B.Cu) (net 16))
 (via (at 162.052 134.874) (size 0.9) (drill 0.4) (layers F.Cu B.Cu) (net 16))
 (segment (start 166.878 133.858) (end 165.862 134.874) (width 0.6096) (layer B.Cu) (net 16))
 (segment (start 172.228 135.702) (end 172.228 134.89) (width 0.6096) (layer F.Cu) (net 6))
 (segment (start 172.228 134.382) (end 172.212 134.366) (width 0.6096) (layer F.Cu) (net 6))
 (via (at 172.212 134.366) (size 0.9) (drill 0.4) (layers F.Cu B.Cu) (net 6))
 (segment (start 172.228 134.89) (end 172.228 134.382) (width 0.6096) (layer F.Cu) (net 6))
 (segment (start 162.052 137.16) (end 162.8755 137.16) (width 0.6096) (layer F.Cu) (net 6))
 (via (at 162.052 137.16) (size 0.9) (drill 0.4) (layers F.Cu B.Cu) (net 6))
 (segment (start 161.2285 137.16) (end 162.052 137.16) (width 0.6096) (layer F.Cu) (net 6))
 (segment (start 168.656 137.16) (end 162.052 137.16) (width 0.6096) (layer B.Cu) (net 6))
 (segment (start 172.212 134.366) (end 170.053 134.366) (width 0.6096) (layer B.Cu) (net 6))
 (segment (start 169.3545 135.0645) (end 169.3545 136.4615) (width 0.6096) (layer B.Cu) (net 6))
 (segment (start 170.053 134.366) (end 169.3545 135.0645) (width 0.6096) (layer B.Cu) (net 6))
 (segment (start 169.3545 136.4615) (end 168.656 137.16) (width 0.6096) (layer B.Cu) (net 6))
 (segment (start 174.228 136.652) (end 174.371 136.652) (width 0.6096) (layer F.Cu) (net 4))
 (segment (start 175.006 137.287) (end 175.891 137.287) (width 0.6096) (layer F.Cu) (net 4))
 (segment (start 174.371 136.652) (end 175.006 137.287) (width 0.6096) (layer F.Cu) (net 4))
 (via (at 174.879 137.922) (size 0.9) (drill 0.4) (layers F.Cu B.Cu) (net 4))
 (segment (start 175.514 137.287) (end 174.879 137.922) (width 0.6096) (layer F.Cu) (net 4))
 (segment (start 175.891 137.287) (end 175.514 137.287) (width 0.6096) (layer F.Cu) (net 4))
 (segment (start 174.879 137.922) (end 175.641 137.16) (width 0.6096) (layer B.Cu) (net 4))
 (via (at 179.578 135.763) (size 0.9) (drill 0.4) (layers F.Cu B.Cu) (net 4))
 (segment (start 178.181 137.16) (end 179.578 135.763) (width 0.6096) (layer B.Cu) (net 4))
 (segment (start 175.641 137.16) (end 178.181 137.16) (width 0.6096) (layer B.Cu) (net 4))
 (segment (start 179.639 135.702) (end 180.61 135.702) (width 0.6096) (layer F.Cu) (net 4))
 (segment (start 179.578 135.763) (end 179.639 135.702) (width 0.6096) (layer F.Cu) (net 4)))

